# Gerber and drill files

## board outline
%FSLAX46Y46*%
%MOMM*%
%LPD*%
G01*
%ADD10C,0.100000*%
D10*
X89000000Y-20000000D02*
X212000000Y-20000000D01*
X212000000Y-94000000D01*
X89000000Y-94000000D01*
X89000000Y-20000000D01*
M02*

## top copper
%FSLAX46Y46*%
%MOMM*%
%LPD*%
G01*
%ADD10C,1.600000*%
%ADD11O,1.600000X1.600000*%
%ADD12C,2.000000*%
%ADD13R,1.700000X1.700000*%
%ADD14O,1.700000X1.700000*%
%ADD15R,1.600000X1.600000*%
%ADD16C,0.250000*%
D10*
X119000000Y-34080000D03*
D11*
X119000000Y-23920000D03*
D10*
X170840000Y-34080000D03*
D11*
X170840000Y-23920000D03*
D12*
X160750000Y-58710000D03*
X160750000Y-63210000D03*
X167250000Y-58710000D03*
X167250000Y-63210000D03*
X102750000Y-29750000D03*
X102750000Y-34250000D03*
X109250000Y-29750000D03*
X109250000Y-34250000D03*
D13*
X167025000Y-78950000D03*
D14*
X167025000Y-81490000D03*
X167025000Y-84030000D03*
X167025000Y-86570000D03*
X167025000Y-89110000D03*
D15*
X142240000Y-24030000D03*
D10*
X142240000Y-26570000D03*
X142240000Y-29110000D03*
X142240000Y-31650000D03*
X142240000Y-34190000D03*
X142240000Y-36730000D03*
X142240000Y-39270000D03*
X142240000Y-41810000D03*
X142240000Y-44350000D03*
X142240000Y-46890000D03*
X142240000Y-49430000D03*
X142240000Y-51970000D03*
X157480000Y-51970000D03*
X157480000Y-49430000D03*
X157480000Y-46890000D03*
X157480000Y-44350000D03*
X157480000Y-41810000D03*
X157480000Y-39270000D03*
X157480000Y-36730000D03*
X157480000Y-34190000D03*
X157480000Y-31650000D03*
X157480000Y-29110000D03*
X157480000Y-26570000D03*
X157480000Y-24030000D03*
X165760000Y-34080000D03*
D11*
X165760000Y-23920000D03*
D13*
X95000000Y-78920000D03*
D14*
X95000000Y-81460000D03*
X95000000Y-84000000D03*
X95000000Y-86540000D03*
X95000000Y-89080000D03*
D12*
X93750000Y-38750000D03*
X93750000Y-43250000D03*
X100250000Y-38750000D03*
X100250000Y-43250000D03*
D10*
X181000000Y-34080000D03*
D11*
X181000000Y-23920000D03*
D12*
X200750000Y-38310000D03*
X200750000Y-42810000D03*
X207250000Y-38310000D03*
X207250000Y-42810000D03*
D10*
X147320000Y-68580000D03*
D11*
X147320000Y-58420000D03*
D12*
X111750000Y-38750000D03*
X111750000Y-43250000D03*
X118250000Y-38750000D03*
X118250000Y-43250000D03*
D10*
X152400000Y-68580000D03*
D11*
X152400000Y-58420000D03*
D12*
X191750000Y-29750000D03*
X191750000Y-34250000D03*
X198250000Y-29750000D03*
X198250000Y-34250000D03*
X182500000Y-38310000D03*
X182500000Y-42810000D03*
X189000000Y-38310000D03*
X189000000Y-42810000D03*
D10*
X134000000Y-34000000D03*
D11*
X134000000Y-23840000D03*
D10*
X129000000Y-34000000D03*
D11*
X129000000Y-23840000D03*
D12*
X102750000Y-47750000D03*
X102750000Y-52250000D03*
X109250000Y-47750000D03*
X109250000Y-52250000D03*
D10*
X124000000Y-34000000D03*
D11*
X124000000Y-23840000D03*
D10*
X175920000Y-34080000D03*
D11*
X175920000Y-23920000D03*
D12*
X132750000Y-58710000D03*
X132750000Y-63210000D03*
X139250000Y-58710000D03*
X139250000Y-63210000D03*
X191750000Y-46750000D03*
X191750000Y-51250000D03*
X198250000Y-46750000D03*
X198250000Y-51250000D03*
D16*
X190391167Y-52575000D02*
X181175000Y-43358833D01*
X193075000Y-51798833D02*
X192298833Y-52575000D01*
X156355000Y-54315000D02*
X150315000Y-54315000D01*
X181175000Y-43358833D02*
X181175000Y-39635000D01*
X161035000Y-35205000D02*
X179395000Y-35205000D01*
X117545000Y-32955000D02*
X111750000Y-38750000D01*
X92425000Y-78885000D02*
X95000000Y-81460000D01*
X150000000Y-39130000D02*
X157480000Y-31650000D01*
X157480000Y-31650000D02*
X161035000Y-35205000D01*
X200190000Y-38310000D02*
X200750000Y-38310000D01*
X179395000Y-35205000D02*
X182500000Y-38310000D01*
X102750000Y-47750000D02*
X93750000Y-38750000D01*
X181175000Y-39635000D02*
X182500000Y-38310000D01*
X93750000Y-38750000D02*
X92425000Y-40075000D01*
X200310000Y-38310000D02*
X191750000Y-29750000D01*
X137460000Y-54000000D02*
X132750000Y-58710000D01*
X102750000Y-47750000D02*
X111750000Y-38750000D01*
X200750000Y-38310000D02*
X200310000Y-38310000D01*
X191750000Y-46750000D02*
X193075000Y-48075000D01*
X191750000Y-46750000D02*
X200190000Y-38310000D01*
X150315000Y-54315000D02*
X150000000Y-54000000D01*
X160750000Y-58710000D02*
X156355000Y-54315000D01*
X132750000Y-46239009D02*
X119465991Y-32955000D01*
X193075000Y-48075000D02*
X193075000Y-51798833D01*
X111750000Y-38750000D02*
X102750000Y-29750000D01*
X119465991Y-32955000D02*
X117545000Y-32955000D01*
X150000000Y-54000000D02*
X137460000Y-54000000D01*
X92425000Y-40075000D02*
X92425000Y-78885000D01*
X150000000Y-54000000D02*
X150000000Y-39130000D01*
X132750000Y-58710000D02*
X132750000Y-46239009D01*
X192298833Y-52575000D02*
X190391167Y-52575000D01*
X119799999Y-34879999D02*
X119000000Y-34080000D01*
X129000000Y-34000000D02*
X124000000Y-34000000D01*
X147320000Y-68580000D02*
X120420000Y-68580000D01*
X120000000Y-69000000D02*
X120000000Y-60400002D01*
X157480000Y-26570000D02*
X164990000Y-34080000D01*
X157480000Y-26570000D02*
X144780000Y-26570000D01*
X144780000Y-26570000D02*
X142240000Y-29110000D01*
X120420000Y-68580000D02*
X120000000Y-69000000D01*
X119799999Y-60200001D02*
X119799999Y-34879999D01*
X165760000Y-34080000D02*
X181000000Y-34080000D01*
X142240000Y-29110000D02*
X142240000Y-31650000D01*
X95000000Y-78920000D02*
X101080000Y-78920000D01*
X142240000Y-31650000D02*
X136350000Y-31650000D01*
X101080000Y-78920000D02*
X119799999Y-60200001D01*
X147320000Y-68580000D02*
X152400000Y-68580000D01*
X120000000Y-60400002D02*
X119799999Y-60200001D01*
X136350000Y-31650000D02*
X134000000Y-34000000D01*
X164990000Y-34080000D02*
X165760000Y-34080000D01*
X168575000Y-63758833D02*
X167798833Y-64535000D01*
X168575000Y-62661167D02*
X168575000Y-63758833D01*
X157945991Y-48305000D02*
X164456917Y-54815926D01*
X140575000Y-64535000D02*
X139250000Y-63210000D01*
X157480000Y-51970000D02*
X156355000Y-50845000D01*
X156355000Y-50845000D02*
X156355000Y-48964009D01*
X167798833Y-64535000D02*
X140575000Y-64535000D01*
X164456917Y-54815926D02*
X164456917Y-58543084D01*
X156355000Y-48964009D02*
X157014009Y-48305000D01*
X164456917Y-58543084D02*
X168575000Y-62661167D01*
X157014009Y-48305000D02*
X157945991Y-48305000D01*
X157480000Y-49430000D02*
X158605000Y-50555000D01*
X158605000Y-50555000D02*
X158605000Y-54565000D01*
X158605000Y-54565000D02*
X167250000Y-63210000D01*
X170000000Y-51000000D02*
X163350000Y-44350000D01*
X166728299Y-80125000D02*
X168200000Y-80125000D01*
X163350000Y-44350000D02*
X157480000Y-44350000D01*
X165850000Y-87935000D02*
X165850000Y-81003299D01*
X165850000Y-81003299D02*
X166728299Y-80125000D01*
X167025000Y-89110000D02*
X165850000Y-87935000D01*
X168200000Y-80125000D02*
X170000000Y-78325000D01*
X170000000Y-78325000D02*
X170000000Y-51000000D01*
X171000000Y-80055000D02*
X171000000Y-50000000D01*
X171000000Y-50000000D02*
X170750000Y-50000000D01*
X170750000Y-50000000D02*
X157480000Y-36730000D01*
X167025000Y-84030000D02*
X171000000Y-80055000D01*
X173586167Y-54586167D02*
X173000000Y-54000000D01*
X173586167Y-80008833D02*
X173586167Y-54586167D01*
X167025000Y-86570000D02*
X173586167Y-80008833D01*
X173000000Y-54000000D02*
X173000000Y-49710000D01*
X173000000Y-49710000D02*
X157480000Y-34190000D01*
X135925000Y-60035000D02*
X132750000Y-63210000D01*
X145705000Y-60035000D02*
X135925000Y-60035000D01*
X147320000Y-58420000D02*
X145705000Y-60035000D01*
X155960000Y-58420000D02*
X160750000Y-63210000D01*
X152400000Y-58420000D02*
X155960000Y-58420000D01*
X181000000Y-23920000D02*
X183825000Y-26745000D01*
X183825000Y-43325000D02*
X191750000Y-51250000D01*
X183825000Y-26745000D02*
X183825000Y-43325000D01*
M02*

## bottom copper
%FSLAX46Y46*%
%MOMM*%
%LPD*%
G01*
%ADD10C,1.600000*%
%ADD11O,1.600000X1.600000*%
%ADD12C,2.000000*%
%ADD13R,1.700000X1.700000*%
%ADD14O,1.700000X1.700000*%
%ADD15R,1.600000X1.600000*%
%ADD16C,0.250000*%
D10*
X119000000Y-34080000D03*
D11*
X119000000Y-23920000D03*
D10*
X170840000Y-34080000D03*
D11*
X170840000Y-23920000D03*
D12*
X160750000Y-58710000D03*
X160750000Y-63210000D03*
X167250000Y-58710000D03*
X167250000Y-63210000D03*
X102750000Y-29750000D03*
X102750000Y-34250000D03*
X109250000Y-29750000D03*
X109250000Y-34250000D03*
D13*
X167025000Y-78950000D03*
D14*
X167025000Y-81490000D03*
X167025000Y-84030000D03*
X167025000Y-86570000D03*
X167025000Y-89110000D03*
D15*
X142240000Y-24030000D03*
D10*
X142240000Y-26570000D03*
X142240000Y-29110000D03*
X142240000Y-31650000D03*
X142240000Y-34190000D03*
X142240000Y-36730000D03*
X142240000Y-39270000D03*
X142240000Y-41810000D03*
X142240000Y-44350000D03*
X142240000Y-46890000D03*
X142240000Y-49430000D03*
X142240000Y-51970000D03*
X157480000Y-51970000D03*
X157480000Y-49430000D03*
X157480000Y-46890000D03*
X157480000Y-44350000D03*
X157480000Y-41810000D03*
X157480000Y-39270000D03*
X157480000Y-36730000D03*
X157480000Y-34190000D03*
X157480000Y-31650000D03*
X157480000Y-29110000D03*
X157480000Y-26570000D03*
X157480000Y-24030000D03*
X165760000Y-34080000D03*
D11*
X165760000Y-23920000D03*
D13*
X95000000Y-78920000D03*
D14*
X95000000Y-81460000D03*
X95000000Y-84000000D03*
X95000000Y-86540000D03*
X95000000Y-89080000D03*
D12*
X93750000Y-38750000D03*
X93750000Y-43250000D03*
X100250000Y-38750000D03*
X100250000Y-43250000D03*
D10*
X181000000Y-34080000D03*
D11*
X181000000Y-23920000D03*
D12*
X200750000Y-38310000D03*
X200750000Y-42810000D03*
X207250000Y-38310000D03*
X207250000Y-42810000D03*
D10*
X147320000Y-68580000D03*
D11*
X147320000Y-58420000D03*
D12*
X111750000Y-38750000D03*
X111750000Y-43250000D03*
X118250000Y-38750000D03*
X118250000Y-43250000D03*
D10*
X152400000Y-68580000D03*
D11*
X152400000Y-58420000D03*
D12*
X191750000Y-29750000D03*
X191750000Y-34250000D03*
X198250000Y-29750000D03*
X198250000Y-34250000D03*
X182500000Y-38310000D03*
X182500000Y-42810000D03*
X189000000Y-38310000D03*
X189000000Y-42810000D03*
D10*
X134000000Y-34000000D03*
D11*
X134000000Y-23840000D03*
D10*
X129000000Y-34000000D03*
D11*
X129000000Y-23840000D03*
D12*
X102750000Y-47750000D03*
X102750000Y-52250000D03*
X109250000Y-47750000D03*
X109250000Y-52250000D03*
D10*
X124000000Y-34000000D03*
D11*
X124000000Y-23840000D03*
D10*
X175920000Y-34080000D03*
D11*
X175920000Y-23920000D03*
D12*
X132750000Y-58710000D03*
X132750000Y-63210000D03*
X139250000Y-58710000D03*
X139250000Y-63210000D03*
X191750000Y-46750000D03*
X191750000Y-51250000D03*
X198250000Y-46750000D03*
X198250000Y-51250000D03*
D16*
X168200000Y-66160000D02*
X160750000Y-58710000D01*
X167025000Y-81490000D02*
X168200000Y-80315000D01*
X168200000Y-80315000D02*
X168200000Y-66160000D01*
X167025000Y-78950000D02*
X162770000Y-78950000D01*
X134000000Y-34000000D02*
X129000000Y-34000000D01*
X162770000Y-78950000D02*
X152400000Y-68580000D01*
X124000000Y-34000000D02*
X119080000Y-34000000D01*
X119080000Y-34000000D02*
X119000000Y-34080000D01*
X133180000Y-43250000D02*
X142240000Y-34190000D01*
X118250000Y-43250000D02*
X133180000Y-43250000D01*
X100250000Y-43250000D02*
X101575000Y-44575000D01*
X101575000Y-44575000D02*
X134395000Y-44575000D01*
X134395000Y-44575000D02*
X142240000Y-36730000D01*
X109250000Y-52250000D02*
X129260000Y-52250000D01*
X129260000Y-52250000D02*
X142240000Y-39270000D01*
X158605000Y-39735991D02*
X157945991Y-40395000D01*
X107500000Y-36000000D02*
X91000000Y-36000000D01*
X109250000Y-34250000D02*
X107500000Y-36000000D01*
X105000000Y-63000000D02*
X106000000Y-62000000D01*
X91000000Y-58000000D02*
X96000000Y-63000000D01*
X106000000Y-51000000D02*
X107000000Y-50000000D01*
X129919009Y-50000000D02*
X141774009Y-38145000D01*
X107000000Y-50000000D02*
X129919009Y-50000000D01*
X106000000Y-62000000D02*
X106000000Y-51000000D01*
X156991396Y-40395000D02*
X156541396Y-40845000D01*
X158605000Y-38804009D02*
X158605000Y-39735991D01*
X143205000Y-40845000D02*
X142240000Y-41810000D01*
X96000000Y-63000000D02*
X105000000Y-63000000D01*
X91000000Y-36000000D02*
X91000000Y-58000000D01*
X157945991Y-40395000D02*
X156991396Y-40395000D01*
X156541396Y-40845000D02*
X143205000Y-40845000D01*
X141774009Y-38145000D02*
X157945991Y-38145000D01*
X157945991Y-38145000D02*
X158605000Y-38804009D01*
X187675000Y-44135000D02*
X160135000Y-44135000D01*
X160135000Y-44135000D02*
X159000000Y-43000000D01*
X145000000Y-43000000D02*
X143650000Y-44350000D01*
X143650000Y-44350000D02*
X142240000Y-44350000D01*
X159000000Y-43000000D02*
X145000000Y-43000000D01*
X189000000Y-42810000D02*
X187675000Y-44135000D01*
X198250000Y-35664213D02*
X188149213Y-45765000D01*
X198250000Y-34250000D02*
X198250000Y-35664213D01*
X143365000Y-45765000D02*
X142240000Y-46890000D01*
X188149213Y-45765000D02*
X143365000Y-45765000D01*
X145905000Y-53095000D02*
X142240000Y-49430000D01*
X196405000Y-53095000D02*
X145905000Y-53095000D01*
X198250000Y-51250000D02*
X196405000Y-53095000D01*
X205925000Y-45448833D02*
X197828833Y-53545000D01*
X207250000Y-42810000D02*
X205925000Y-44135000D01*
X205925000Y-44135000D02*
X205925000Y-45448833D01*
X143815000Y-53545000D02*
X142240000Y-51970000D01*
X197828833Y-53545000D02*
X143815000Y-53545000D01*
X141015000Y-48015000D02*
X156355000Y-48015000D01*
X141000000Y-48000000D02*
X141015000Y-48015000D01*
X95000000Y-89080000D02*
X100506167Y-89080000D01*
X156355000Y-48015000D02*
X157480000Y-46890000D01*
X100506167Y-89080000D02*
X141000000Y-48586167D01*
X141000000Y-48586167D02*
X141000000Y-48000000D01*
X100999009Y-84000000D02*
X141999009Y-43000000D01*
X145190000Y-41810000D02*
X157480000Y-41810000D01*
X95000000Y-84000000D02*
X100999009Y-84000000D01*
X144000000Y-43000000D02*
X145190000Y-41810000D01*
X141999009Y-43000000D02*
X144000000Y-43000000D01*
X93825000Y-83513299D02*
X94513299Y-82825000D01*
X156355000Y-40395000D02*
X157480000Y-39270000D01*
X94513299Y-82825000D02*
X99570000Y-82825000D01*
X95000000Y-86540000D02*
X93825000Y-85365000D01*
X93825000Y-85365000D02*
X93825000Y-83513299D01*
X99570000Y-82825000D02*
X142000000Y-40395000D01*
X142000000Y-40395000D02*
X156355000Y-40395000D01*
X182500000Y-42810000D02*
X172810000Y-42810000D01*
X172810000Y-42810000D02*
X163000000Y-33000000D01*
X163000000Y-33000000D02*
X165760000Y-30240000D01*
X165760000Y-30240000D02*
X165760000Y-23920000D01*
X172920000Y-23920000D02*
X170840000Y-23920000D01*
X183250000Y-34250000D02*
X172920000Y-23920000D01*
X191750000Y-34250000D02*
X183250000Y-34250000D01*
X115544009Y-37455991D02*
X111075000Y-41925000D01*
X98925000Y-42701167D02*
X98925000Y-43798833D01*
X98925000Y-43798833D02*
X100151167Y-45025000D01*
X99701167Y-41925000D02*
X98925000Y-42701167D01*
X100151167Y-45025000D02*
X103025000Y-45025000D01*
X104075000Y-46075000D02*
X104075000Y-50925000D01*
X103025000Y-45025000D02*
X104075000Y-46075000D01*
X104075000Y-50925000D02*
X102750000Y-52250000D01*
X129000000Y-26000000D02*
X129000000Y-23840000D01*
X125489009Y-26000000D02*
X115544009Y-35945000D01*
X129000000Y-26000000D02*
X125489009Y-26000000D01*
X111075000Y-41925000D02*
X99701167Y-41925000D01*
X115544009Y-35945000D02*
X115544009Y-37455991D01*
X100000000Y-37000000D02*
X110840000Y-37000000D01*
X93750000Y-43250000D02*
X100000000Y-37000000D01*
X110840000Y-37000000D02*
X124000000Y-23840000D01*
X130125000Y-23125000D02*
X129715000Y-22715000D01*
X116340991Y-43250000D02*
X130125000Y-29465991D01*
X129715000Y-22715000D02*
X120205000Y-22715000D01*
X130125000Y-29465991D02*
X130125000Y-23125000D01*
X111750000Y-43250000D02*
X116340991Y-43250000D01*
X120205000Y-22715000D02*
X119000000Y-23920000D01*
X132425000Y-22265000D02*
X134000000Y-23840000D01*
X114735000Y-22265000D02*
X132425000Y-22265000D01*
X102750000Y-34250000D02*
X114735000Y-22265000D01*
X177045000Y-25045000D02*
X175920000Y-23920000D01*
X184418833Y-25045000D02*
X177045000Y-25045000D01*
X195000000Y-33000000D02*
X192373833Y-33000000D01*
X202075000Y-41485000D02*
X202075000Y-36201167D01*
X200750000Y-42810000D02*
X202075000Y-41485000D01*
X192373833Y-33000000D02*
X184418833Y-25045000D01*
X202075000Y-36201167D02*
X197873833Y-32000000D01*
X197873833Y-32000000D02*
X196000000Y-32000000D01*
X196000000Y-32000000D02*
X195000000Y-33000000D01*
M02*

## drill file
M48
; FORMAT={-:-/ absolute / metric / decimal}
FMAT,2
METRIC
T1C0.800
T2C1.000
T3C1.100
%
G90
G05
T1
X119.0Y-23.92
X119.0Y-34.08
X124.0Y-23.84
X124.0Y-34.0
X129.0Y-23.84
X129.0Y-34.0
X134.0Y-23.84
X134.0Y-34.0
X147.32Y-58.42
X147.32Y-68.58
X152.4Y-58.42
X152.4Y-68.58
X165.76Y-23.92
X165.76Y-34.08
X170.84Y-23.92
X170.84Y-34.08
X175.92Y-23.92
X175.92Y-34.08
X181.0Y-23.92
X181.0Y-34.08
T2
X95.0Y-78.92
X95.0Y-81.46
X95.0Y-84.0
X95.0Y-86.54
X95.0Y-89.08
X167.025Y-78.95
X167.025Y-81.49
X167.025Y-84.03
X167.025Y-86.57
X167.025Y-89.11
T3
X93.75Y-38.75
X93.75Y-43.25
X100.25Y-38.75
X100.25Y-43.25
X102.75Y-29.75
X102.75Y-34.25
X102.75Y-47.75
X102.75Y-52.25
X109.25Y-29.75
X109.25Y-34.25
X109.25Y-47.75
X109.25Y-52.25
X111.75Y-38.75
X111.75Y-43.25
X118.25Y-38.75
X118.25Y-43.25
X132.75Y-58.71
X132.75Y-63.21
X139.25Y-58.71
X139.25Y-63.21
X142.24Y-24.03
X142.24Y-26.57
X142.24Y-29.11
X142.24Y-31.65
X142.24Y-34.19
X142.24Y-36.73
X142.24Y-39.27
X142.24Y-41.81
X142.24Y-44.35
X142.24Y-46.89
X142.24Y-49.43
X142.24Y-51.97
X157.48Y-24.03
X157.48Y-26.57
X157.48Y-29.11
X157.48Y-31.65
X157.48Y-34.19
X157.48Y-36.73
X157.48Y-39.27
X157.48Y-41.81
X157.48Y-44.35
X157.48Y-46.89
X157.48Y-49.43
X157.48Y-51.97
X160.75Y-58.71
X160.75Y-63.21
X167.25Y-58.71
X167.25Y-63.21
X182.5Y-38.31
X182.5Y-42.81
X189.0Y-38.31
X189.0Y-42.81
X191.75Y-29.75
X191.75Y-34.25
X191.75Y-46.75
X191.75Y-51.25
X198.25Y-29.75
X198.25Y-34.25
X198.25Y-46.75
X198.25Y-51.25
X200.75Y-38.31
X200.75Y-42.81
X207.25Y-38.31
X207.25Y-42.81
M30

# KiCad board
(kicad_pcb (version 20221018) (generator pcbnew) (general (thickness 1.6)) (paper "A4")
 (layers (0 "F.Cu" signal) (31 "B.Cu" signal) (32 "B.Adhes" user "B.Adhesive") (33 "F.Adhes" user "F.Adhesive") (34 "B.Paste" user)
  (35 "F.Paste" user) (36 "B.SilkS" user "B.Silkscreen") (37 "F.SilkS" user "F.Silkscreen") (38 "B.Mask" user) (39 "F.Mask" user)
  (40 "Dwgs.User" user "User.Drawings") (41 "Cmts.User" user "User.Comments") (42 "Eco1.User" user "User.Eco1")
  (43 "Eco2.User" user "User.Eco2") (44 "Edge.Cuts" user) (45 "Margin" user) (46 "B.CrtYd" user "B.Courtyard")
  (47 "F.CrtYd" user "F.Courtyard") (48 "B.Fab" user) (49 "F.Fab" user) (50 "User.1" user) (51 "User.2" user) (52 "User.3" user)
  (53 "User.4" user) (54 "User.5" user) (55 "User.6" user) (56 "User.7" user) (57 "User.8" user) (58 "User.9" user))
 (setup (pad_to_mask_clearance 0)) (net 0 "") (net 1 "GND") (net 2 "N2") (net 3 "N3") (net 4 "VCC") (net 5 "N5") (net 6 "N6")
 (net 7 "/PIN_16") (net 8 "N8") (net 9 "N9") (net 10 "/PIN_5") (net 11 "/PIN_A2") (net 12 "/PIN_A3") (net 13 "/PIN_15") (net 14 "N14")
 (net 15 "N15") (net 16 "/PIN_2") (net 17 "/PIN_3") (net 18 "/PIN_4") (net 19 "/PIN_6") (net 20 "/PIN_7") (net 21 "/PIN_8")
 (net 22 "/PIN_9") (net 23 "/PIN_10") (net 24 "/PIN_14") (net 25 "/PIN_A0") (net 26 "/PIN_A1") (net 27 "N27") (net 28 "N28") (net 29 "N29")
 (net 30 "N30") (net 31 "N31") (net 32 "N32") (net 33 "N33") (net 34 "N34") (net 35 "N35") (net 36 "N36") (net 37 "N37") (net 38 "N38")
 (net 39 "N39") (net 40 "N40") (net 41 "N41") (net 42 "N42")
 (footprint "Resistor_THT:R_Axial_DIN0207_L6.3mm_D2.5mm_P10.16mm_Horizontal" (layer "F.Cu") (at 119 34.08 90)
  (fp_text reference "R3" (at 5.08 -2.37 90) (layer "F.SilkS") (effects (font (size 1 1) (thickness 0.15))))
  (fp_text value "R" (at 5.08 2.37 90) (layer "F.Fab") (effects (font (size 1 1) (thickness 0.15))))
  (pad "1" thru_hole circle (at 0 0 90) (size 1.6 1.6) (drill 0.8) (layers "*.Cu" "*.Mask") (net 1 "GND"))
  (pad "2" thru_hole oval (at 10.16 0 90) (size 1.6 1.6) (drill 0.8) (layers "*.Cu" "*.Mask") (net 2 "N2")))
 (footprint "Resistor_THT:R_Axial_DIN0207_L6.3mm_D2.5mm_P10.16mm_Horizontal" (layer "F.Cu") (at 170.84 34.08 90)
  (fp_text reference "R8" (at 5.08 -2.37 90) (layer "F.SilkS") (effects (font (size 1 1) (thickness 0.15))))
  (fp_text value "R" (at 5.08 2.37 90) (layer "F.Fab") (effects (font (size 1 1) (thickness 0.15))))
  (pad "1" thru_hole circle (at 0 0 90) (size 1.6 1.6) (drill 0.8) (layers "*.Cu" "*.Mask") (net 1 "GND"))
  (pad "2" thru_hole oval (at 10.16 0 90) (size 1.6 1.6) (drill 0.8) (layers "*.Cu" "*.Mask") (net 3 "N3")))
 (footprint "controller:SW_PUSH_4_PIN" (layer "F.Cu") (at 160.75 58.71)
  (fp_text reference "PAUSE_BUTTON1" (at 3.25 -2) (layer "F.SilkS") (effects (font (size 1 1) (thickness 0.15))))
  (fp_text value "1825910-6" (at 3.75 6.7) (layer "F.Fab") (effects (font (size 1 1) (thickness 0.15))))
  (pad "1" thru_hole circle (at 0 0 90) (size 2 2) (drill 1.1) (layers "*.Cu" "*.Mask") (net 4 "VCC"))
  (pad "2" thru_hole circle (at 0 4.5 90) (size 2 2) (drill 1.1) (layers "*.Cu" "*.Mask") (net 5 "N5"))
  (pad "3" thru_hole circle (at 6.5 0 90) (size 2 2) (drill 1.1) (layers "*.Cu" "*.Mask") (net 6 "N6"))
  (pad "4" thru_hole circle (at 6.5 4.5 90) (size 2 2) (drill 1.1) (layers "*.Cu" "*.Mask") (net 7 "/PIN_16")))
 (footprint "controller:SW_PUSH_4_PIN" (layer "F.Cu") (at 102.75 29.75)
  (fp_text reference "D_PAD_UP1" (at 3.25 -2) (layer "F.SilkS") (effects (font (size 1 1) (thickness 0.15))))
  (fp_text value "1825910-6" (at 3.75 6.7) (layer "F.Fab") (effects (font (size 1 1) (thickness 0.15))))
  (pad "1" thru_hole circle (at 0 0 90) (size 2 2) (drill 1.1) (layers "*.Cu" "*.Mask") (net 4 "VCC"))
  (pad "2" thru_hole circle (at 0 4.5 90) (size 2 2) (drill 1.1) (layers "*.Cu" "*.Mask") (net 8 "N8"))
  (pad "3" thru_hole circle (at 6.5 0 90) (size 2 2) (drill 1.1) (layers "*.Cu" "*.Mask") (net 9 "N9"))
  (pad "4" thru_hole circle (at 6.5 4.5 90) (size 2 2) (drill 1.1) (layers "*.Cu" "*.Mask") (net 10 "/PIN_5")))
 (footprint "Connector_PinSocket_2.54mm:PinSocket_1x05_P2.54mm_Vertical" (layer "F.Cu") (at 167.025 78.95)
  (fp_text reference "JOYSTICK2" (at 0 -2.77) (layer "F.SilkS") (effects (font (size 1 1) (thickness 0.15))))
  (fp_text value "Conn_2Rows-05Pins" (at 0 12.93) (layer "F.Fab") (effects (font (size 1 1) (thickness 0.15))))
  (pad "1" thru_hole rect (at 0 0) (size 1.7 1.7) (drill 1) (layers "*.Cu" "*.Mask") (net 1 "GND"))
  (pad "2" thru_hole oval (at 0 2.54) (size 1.7 1.7) (drill 1) (layers "*.Cu" "*.Mask") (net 4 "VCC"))
  (pad "3" thru_hole oval (at 0 5.08) (size 1.7 1.7) (drill 1) (layers "*.Cu" "*.Mask") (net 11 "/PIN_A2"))
  (pad "4" thru_hole oval (at 0 7.62) (size 1.7 1.7) (drill 1) (layers "*.Cu" "*.Mask") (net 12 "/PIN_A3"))
  (pad "5" thru_hole oval (at 0 10.16) (size 1.7 1.7) (drill 1) (layers "*.Cu" "*.Mask") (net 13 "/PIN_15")))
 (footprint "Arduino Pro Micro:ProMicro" (layer "F.Cu") (at 149.86 38 -90)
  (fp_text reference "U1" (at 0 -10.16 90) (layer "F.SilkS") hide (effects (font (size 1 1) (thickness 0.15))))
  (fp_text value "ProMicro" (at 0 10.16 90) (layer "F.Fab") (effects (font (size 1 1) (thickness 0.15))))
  (pad "1" thru_hole rect (at -13.97 7.62 270) (size 1.6 1.6) (drill 1.1) (layers "*.Cu" "*.Mask" "F.SilkS") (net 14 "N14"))
  (pad "2" thru_hole circle (at -11.43 7.62 270) (size 1.6 1.6) (drill 1.1) (layers "*.Cu" "*.Mask" "F.SilkS") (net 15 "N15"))
  (pad "3" thru_hole circle (at -8.89 7.62 270) (size 1.6 1.6) (drill 1.1) (layers "*.Cu" "*.Mask" "F.SilkS") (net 1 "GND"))
  (pad "4" thru_hole circle (at -6.35 7.62 270) (size 1.6 1.6) (drill 1.1) (layers "*.Cu" "*.Mask" "F.SilkS") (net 1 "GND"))
  (pad "5" thru_hole circle (at -3.81 7.62 270) (size 1.6 1.6) (drill 1.1) (layers "*.Cu" "*.Mask" "F.SilkS") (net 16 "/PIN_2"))
  (pad "6" thru_hole circle (at -1.27 7.62 270) (size 1.6 1.6) (drill 1.1) (layers "*.Cu" "*.Mask" "F.SilkS") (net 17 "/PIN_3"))
  (pad "7" thru_hole circle (at 1.27 7.62 270) (size 1.6 1.6) (drill 1.1) (layers "*.Cu" "*.Mask" "F.SilkS") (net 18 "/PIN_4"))
  (pad "8" thru_hole circle (at 3.81 7.62 270) (size 1.6 1.6) (drill 1.1) (layers "*.Cu" "*.Mask" "F.SilkS") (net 10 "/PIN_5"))
  (pad "9" thru_hole circle (at 6.35 7.62 270) (size 1.6 1.6) (drill 1.1) (layers "*.Cu" "*.Mask" "F.SilkS") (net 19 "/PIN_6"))
  (pad "10" thru_hole circle (at 8.89 7.62 270) (size 1.6 1.6) (drill 1.1) (layers "*.Cu" "*.Mask" "F.SilkS") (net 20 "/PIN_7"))
  (pad "11" thru_hole circle (at 11.43 7.62 270) (size 1.6 1.6) (drill 1.1) (layers "*.Cu" "*.Mask" "F.SilkS") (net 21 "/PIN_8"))
  (pad "12" thru_hole circle (at 13.97 7.62 270) (size 1.6 1.6) (drill 1.1) (layers "*.Cu" "*.Mask" "F.SilkS") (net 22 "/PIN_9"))
  (pad "13" thru_hole circle (at 13.97 -7.62 270) (size 1.6 1.6) (drill 1.1) (layers "*.Cu" "*.Mask" "F.SilkS") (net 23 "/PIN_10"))
  (pad "14" thru_hole circle (at 11.43 -7.62 270) (size 1.6 1.6) (drill 1.1) (layers "*.Cu" "*.Mask" "F.SilkS") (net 7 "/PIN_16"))
  (pad "15" thru_hole circle (at 8.89 -7.62 270) (size 1.6 1.6) (drill 1.1) (layers "*.Cu" "*.Mask" "F.SilkS") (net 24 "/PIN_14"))
  (pad "16" thru_hole circle (at 6.35 -7.62 270) (size 1.6 1.6) (drill 1.1) (layers "*.Cu" "*.Mask" "F.SilkS") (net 13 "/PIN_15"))
  (pad "17" thru_hole circle (at 3.81 -7.62 270) (size 1.6 1.6) (drill 1.1) (layers "*.Cu" "*.Mask" "F.SilkS") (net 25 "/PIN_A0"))
  (pad "18" thru_hole circle (at 1.27 -7.62 270) (size 1.6 1.6) (drill 1.1) (layers "*.Cu" "*.Mask" "F.SilkS") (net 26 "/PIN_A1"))
  (pad "19" thru_hole circle (at -1.27 -7.62 270) (size 1.6 1.6) (drill 1.1) (layers "*.Cu" "*.Mask" "F.SilkS") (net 11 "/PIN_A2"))
  (pad "20" thru_hole circle (at -3.81 -7.62 270) (size 1.6 1.6) (drill 1.1) (layers "*.Cu" "*.Mask" "F.SilkS") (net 12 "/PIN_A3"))
  (pad "21" thru_hole circle (at -6.35 -7.62 270) (size 1.6 1.6) (drill 1.1) (layers "*.Cu" "*.Mask" "F.SilkS") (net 4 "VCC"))
  (pad "22" thru_hole circle (at -8.89 -7.62 270) (size 1.6 1.6) (drill 1.1) (layers "*.Cu" "*.Mask" "F.SilkS") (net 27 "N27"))
  (pad "23" thru_hole circle (at -11.43 -7.62 270) (size 1.6 1.6) (drill 1.1) (layers "*.Cu" "*.Mask" "F.SilkS") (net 1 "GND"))
  (pad "24" thru_hole circle (at -13.97 -7.62 270) (size 1.6 1.6) (drill 1.1) (layers "*.Cu" "*.Mask" "F.SilkS") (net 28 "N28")))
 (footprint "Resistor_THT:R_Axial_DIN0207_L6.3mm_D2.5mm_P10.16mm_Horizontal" (layer "F.Cu") (at 165.76 34.08 90)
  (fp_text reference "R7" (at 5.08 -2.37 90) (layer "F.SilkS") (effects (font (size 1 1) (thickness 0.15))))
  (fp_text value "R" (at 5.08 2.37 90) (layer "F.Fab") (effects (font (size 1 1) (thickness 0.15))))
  (pad "1" thru_hole circle (at 0 0 90) (size 1.6 1.6) (drill 0.8) (layers "*.Cu" "*.Mask") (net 1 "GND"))
  (pad "2" thru_hole oval (at 10.16 0 90) (size 1.6 1.6) (drill 0.8) (layers "*.Cu" "*.Mask") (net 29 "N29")))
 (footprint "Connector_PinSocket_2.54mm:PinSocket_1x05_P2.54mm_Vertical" (layer "F.Cu") (at 95 78.92)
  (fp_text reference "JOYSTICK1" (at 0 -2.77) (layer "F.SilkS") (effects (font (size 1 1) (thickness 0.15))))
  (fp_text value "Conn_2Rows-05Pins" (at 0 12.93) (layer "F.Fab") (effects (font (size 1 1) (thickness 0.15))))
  (pad "1" thru_hole rect (at 0 0) (size 1.7 1.7) (drill 1) (layers "*.Cu" "*.Mask") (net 1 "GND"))
  (pad "2" thru_hole oval (at 0 2.54) (size 1.7 1.7) (drill 1) (layers "*.Cu" "*.Mask") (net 4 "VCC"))
  (pad "3" thru_hole oval (at 0 5.08) (size 1.7 1.7) (drill 1) (layers "*.Cu" "*.Mask") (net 25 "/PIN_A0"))
  (pad "4" thru_hole oval (at 0 7.62) (size 1.7 1.7) (drill 1) (layers "*.Cu" "*.Mask") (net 26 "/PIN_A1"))
  (pad "5" thru_hole oval (at 0 10.16) (size 1.7 1.7) (drill 1) (layers "*.Cu" "*.Mask") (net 24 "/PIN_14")))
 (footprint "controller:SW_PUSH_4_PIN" (layer "F.Cu") (at 93.75 38.75)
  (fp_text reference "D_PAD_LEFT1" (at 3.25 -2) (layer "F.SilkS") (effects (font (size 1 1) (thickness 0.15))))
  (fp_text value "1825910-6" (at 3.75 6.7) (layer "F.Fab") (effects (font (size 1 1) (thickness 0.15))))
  (pad "1" thru_hole circle (at 0 0 90) (size 2 2) (drill 1.1) (layers "*.Cu" "*.Mask") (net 4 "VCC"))
  (pad "2" thru_hole circle (at 0 4.5 90) (size 2 2) (drill 1.1) (layers "*.Cu" "*.Mask") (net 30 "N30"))
  (pad "3" thru_hole circle (at 6.5 0 90) (size 2 2) (drill 1.1) (layers "*.Cu" "*.Mask") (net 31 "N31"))
  (pad "4" thru_hole circle (at 6.5 4.5 90) (size 2 2) (drill 1.1) (layers "*.Cu" "*.Mask") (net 17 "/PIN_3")))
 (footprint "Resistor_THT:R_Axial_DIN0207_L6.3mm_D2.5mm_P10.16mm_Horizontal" (layer "F.Cu") (at 181 34.08 90)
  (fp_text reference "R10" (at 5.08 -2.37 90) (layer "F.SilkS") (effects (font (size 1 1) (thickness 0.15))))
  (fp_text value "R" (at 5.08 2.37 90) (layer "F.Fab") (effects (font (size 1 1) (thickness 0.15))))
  (pad "1" thru_hole circle (at 0 0 90) (size 1.6 1.6) (drill 0.8) (layers "*.Cu" "*.Mask") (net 1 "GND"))
  (pad "2" thru_hole oval (at 10.16 0 90) (size 1.6 1.6) (drill 0.8) (layers "*.Cu" "*.Mask") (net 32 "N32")))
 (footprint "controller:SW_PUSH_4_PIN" (layer "F.Cu") (at 200.75 38.31)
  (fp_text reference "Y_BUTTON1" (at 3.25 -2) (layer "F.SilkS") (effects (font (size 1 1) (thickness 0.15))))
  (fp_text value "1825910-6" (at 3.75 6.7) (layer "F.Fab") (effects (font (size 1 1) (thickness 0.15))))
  (pad "1" thru_hole circle (at 0 0 90) (size 2 2) (drill 1.1) (layers "*.Cu" "*.Mask") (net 4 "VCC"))
  (pad "2" thru_hole circle (at 0 4.5 90) (size 2 2) (drill 1.1) (layers "*.Cu" "*.Mask") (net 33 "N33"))
  (pad "3" thru_hole circle (at 6.5 0 90) (size 2 2) (drill 1.1) (layers "*.Cu" "*.Mask") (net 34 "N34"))
  (pad "4" thru_hole circle (at 6.5 4.5 90) (size 2 2) (drill 1.1) (layers "*.Cu" "*.Mask") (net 22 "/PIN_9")))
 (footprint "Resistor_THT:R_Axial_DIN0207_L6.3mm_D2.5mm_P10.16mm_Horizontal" (layer "F.Cu") (at 147.32 68.58 90)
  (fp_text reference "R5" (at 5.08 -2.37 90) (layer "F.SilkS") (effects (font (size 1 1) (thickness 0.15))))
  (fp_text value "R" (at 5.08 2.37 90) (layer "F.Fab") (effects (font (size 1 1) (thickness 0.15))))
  (pad "1" thru_hole circle (at 0 0 90) (size 1.6 1.6) (drill 0.8) (layers "*.Cu" "*.Mask") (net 1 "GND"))
  (pad "2" thru_hole oval (at 10.16 0 90) (size 1.6 1.6) (drill 0.8) (layers "*.Cu" "*.Mask") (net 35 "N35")))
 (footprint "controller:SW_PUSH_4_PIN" (layer "F.Cu") (at 111.75 38.75)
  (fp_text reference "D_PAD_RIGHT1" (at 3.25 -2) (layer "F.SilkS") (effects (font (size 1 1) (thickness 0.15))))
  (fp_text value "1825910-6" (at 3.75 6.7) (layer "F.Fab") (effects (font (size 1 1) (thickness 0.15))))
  (pad "1" thru_hole circle (at 0 0 90) (size 2 2) (drill 1.1) (layers "*.Cu" "*.Mask") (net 4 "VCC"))
  (pad "2" thru_hole circle (at 0 4.5 90) (size 2 2) (drill 1.1) (layers "*.Cu" "*.Mask") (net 2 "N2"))
  (pad "3" thru_hole circle (at 6.5 0 90) (size 2 2) (drill 1.1) (layers "*.Cu" "*.Mask") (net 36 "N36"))
  (pad "4" thru_hole circle (at 6.5 4.5 90) (size 2 2) (drill 1.1) (layers "*.Cu" "*.Mask") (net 16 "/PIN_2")))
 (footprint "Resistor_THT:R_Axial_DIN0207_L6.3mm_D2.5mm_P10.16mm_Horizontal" (layer "F.Cu") (at 152.4 68.58 90)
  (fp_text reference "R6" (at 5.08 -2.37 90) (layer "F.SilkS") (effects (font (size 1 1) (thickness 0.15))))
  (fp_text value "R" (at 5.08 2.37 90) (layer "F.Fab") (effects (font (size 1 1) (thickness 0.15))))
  (pad "1" thru_hole circle (at 0 0 90) (size 1.6 1.6) (drill 0.8) (layers "*.Cu" "*.Mask") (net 1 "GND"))
  (pad "2" thru_hole oval (at 10.16 0 90) (size 1.6 1.6) (drill 0.8) (layers "*.Cu" "*.Mask") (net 5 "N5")))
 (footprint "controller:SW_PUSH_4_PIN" (layer "F.Cu") (at 191.75 29.75)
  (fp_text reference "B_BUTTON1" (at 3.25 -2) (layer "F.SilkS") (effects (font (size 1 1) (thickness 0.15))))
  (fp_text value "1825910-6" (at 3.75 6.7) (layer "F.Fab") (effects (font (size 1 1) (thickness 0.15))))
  (pad "1" thru_hole circle (at 0 0 90) (size 2 2) (drill 1.1) (layers "*.Cu" "*.Mask") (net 4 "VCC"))
  (pad "2" thru_hole circle (at 0 4.5 90) (size 2 2) (drill 1.1) (layers "*.Cu" "*.Mask") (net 3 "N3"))
  (pad "3" thru_hole circle (at 6.5 0 90) (size 2 2) (drill 1.1) (layers "*.Cu" "*.Mask") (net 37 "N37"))
  (pad "4" thru_hole circle (at 6.5 4.5 90) (size 2 2) (drill 1.1) (layers "*.Cu" "*.Mask") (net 20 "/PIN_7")))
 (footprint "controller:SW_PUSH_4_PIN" (layer "F.Cu") (at 182.5 38.31)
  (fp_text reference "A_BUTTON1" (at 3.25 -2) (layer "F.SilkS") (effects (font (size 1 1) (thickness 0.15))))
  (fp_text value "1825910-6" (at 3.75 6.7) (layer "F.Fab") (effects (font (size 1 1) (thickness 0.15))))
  (pad "1" thru_hole circle (at 0 0 90) (size 2 2) (drill 1.1) (layers "*.Cu" "*.Mask") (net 4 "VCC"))
  (pad "2" thru_hole circle (at 0 4.5 90) (size 2 2) (drill 1.1) (layers "*.Cu" "*.Mask") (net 29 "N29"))
  (pad "3" thru_hole circle (at 6.5 0 90) (size 2 2) (drill 1.1) (layers "*.Cu" "*.Mask") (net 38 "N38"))
  (pad "4" thru_hole circle (at 6.5 4.5 90) (size 2 2) (drill 1.1) (layers "*.Cu" "*.Mask") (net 19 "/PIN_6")))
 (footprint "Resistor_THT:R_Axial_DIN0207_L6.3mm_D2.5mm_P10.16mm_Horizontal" (layer "F.Cu") (at 134 34 90)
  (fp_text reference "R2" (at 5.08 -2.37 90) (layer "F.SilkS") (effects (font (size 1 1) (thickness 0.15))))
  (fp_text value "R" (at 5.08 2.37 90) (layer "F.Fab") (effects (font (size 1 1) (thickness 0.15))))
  (pad "1" thru_hole circle (at 0 0 90) (size 1.6 1.6) (drill 0.8) (layers "*.Cu" "*.Mask") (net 1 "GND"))
  (pad "2" thru_hole oval (at 10.16 0 90) (size 1.6 1.6) (drill 0.8) (layers "*.Cu" "*.Mask") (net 8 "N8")))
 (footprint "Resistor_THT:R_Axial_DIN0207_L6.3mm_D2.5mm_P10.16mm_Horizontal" (layer "F.Cu") (at 129 34 90)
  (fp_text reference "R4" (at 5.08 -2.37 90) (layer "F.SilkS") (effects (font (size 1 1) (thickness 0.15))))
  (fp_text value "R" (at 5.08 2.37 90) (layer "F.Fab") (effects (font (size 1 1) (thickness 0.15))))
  (pad "1" thru_hole circle (at 0 0 90) (size 1.6 1.6) (drill 0.8) (layers "*.Cu" "*.Mask") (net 1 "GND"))
  (pad "2" thru_hole oval (at 10.16 0 90) (size 1.6 1.6) (drill 0.8) (layers "*.Cu" "*.Mask") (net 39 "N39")))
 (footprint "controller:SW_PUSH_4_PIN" (layer "F.Cu") (at 102.75 47.75)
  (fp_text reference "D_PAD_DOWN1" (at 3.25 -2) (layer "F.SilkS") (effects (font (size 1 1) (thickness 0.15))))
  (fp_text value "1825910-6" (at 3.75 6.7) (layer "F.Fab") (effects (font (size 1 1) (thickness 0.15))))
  (pad "1" thru_hole circle (at 0 0 90) (size 2 2) (drill 1.1) (layers "*.Cu" "*.Mask") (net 4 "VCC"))
  (pad "2" thru_hole circle (at 0 4.5 90) (size 2 2) (drill 1.1) (layers "*.Cu" "*.Mask") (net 39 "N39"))
  (pad "3" thru_hole circle (at 6.5 0 90) (size 2 2) (drill 1.1) (layers "*.Cu" "*.Mask") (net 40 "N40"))
  (pad "4" thru_hole circle (at 6.5 4.5 90) (size 2 2) (drill 1.1) (layers "*.Cu" "*.Mask") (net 18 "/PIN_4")))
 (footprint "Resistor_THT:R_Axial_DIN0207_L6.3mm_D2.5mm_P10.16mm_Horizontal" (layer "F.Cu") (at 124 34 90)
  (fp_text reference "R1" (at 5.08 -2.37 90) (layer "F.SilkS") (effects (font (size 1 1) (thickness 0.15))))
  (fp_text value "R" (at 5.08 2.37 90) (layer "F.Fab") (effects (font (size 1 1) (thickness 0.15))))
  (pad "1" thru_hole circle (at 0 0 90) (size 1.6 1.6) (drill 0.8) (layers "*.Cu" "*.Mask") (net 1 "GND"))
  (pad "2" thru_hole oval (at 10.16 0 90) (size 1.6 1.6) (drill 0.8) (layers "*.Cu" "*.Mask") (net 30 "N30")))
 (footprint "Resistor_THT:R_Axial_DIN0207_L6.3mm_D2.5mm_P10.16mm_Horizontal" (layer "F.Cu") (at 175.92 34.08 90)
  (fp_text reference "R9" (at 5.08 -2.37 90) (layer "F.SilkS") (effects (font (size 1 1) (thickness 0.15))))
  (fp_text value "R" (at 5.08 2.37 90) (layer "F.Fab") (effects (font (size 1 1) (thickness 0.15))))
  (pad "1" thru_hole circle (at 0 0 90) (size 1.6 1.6) (drill 0.8) (layers "*.Cu" "*.Mask") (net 1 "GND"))
  (pad "2" thru_hole oval (at 10.16 0 90) (size 1.6 1.6) (drill 0.8) (layers "*.Cu" "*.Mask") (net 33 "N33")))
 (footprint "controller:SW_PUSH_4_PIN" (layer "F.Cu") (at 132.75 58.71)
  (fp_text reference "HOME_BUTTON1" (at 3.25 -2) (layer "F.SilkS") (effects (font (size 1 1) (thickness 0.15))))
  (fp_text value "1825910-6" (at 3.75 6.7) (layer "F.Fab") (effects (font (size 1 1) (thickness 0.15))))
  (pad "1" thru_hole circle (at 0 0 90) (size 2 2) (drill 1.1) (layers "*.Cu" "*.Mask") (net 4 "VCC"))
  (pad "2" thru_hole circle (at 0 4.5 90) (size 2 2) (drill 1.1) (layers "*.Cu" "*.Mask") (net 35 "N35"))
  (pad "3" thru_hole circle (at 6.5 0 90) (size 2 2) (drill 1.1) (layers "*.Cu" "*.Mask") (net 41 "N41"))
  (pad "4" thru_hole circle (at 6.5 4.5 90) (size 2 2) (drill 1.1) (layers "*.Cu" "*.Mask") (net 23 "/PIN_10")))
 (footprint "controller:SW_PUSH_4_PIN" (layer "F.Cu") (at 191.75 46.75)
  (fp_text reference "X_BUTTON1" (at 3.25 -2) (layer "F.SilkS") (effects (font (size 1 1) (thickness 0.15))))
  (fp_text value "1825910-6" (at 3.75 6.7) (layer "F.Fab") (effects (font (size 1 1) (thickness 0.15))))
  (pad "1" thru_hole circle (at 0 0 90) (size 2 2) (drill 1.1) (layers "*.Cu" "*.Mask") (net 4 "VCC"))
  (pad "2" thru_hole circle (at 0 4.5 90) (size 2 2) (drill 1.1) (layers "*.Cu" "*.Mask") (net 32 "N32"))
  (pad "3" thru_hole circle (at 6.5 0 90) (size 2 2) (drill 1.1) (layers "*.Cu" "*.Mask") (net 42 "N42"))
  (pad "4" thru_hole circle (at 6.5 4.5 90) (size 2 2) (drill 1.1) (layers "*.Cu" "*.Mask") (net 21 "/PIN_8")))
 (gr_rect (start 89 20) (end 212 94) (stroke (width 0.1) (type default)) (fill none) (layer "Edge.Cuts"))
 (segment (start 190.391167 52.575) (end 181.175 43.358833) (width 0.25) (layer "F.Cu") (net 4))
 (segment (start 193.075 51.798833) (end 192.298833 52.575) (width 0.25) (layer "F.Cu") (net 4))
 (segment (start 156.355 54.315) (end 150.315 54.315) (width 0.25) (layer "F.Cu") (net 4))
 (segment (start 181.175 43.358833) (end 181.175 39.635) (width 0.25) (layer "F.Cu") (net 4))
 (segment (start 161.035 35.205) (end 179.395 35.205) (width 0.25) (layer "F.Cu") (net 4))
 (segment (start 117.545 32.955) (end 111.75 38.75) (width 0.25) (layer "F.Cu") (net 4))
 (segment (start 92.425 78.885) (end 95 81.46) (width 0.25) (layer "F.Cu") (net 4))
 (segment (start 150 39.13) (end 157.48 31.65) (width 0.25) (layer "F.Cu") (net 4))
 (segment (start 157.48 31.65) (end 161.035 35.205) (width 0.25) (layer "F.Cu") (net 4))
 (segment (start 200.19 38.31) (end 200.75 38.31) (width 0.25) (layer "F.Cu") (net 4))
 (segment (start 179.395 35.205) (end 182.5 38.31) (width 0.25) (layer "F.Cu") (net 4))
 (segment (start 102.75 47.75) (end 93.75 38.75) (width 0.25) (layer "F.Cu") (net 4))
 (segment (start 181.175 39.635) (end 182.5 38.31) (width 0.25) (layer "F.Cu") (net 4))
 (segment (start 93.75 38.75) (end 92.425 40.075) (width 0.25) (layer "F.Cu") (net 4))
 (segment (start 200.31 38.31) (end 191.75 29.75) (width 0.25) (layer "F.Cu") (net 4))
 (segment (start 137.46 54) (end 132.75 58.71) (width 0.25) (layer "F.Cu") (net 4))
 (segment (start 102.75 47.75) (end 111.75 38.75) (width 0.25) (layer "F.Cu") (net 4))
 (segment (start 200.75 38.31) (end 200.31 38.31) (width 0.25) (layer "F.Cu") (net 4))
 (segment (start 191.75 46.75) (end 193.075 48.075) (width 0.25) (layer "F.Cu") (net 4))
 (segment (start 191.75 46.75) (end 200.19 38.31) (width 0.25) (layer "F.Cu") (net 4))
 (segment (start 150.315 54.315) (end 150 54) (width 0.25) (layer "F.Cu") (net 4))
 (segment (start 160.75 58.71) (end 156.355 54.315) (width 0.25) (layer "F.Cu") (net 4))
 (segment (start 132.75 46.239009) (end 119.465991 32.955) (width 0.25) (layer "F.Cu") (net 4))
 (segment (start 193.075 48.075) (end 193.075 51.798833) (width 0.25) (layer "F.Cu") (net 4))
 (segment (start 111.75 38.75) (end 102.75 29.75) (width 0.25) (layer "F.Cu") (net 4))
 (segment (start 119.465991 32.955) (end 117.545 32.955) (width 0.25) (layer "F.Cu") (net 4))
 (segment (start 150 54) (end 137.46 54) (width 0.25) (layer "F.Cu") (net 4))
 (segment (start 92.425 40.075) (end 92.425 78.885) (width 0.25) (layer "F.Cu") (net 4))
 (segment (start 150 54) (end 150 39.13) (width 0.25) (layer "F.Cu") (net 4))
 (segment (start 132.75 58.71) (end 132.75 46.239009) (width 0.25) (layer "F.Cu") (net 4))
 (segment (start 192.298833 52.575) (end 190.391167 52.575) (width 0.25) (layer "F.Cu") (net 4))
 (segment (start 168.2 66.16) (end 160.75 58.71) (width 0.25) (layer "B.Cu") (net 4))
 (segment (start 167.025 81.49) (end 168.2 80.315) (width 0.25) (layer "B.Cu") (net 4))
 (segment (start 168.2 80.315) (end 168.2 66.16) (width 0.25) (layer "B.Cu") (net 4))
 (segment (start 119.799999 34.879999) (end 119 34.08) (width 0.25) (layer "F.Cu") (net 1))
 (segment (start 129 34) (end 124 34) (width 0.25) (layer "F.Cu") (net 1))
 (segment (start 147.32 68.58) (end 120.42 68.58) (width 0.25) (layer "F.Cu") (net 1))
 (segment (start 120 69) (end 120 60.400002) (width 0.25) (layer "F.Cu") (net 1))
 (segment (start 157.48 26.57) (end 164.99 34.08) (width 0.25) (layer "F.Cu") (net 1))
 (segment (start 157.48 26.57) (end 144.78 26.57) (width 0.25) (layer "F.Cu") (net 1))
 (segment (start 144.78 26.57) (end 142.24 29.11) (width 0.25) (layer "F.Cu") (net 1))
 (segment (start 120.42 68.58) (end 120 69) (width 0.25) (layer "F.Cu") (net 1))
 (segment (start 119.799999 60.200001) (end 119.799999 34.879999) (width 0.25) (layer "F.Cu") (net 1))
 (segment (start 165.76 34.08) (end 181 34.08) (width 0.25) (layer "F.Cu") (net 1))
 (segment (start 142.24 29.11) (end 142.24 31.65) (width 0.25) (layer "F.Cu") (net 1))
 (segment (start 95 78.92) (end 101.08 78.92) (width 0.25) (layer "F.Cu") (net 1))
 (segment (start 142.24 31.65) (end 136.35 31.65) (width 0.25) (layer "F.Cu") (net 1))
 (segment (start 101.08 78.92) (end 119.799999 60.200001) (width 0.25) (layer "F.Cu") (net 1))
 (segment (start 147.32 68.58) (end 152.4 68.58) (width 0.25) (layer "F.Cu") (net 1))
 (segment (start 120 60.400002) (end 119.799999 60.200001) (width 0.25) (layer "F.Cu") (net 1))
 (segment (start 136.35 31.65) (end 134 34) (width 0.25) (layer "F.Cu") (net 1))
 (segment (start 164.99 34.08) (end 165.76 34.08) (width 0.25) (layer "F.Cu") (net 1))
 (segment (start 167.025 78.95) (end 162.77 78.95) (width 0.25) (layer "B.Cu") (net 1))
 (segment (start 134 34) (end 129 34) (width 0.25) (layer "B.Cu") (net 1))
 (segment (start 162.77 78.95) (end 152.4 68.58) (width 0.25) (layer "B.Cu") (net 1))
 (segment (start 124 34) (end 119.08 34) (width 0.25) (layer "B.Cu") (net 1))
 (segment (start 119.08 34) (end 119 34.08) (width 0.25) (layer "B.Cu") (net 1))
 (segment (start 133.18 43.25) (end 142.24 34.19) (width 0.25) (layer "B.Cu") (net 16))
 (segment (start 118.25 43.25) (end 133.18 43.25) (width 0.25) (layer "B.Cu") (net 16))
 (segment (start 100.25 43.25) (end 101.575 44.575) (width 0.25) (layer "B.Cu") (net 17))
 (segment (start 101.575 44.575) (end 134.395 44.575) (width 0.25) (layer "B.Cu") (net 17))
 (segment (start 134.395 44.575) (end 142.24 36.73) (width 0.25) (layer "B.Cu") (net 17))
 (segment (start 109.25 52.25) (end 129.26 52.25) (width 0.25) (layer "B.Cu") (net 18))
 (segment (start 129.26 52.25) (end 142.24 39.27) (width 0.25) (layer "B.Cu") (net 18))
 (segment (start 158.605 39.735991) (end 157.945991 40.395) (width 0.25) (layer "B.Cu") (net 10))
 (segment (start 107.5 36) (end 91 36) (width 0.25) (layer "B.Cu") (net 10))
 (segment (start 109.25 34.25) (end 107.5 36) (width 0.25) (layer "B.Cu") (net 10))
 (segment (start 105 63) (end 106 62) (width 0.25) (layer "B.Cu") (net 10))
 (segment (start 91 58) (end 96 63) (width 0.25) (layer "B.Cu") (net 10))
 (segment (start 106 51) (end 107 50) (width 0.25) (layer "B.Cu") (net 10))
 (segment (start 129.919009 50) (end 141.774009 38.145) (width 0.25) (layer "B.Cu") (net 10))
 (segment (start 107 50) (end 129.919009 50) (width 0.25) (layer "B.Cu") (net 10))
 (segment (start 106 62) (end 106 51) (width 0.25) (layer "B.Cu") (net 10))
 (segment (start 156.991396 40.395) (end 156.541396 40.845) (width 0.25) (layer "B.Cu") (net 10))
 (segment (start 158.605 38.804009) (end 158.605 39.735991) (width 0.25) (layer "B.Cu") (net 10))
 (segment (start 143.205 40.845) (end 142.24 41.81) (width 0.25) (layer "B.Cu") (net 10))
 (segment (start 96 63) (end 105 63) (width 0.25) (layer "B.Cu") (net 10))
 (segment (start 91 36) (end 91 58) (width 0.25) (layer "B.Cu") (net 10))
 (segment (start 157.945991 40.395) (end 156.991396 40.395) (width 0.25) (layer "B.Cu") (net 10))
 (segment (start 156.541396 40.845) (end 143.205 40.845) (width 0.25) (layer "B.Cu") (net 10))
 (segment (start 141.774009 38.145) (end 157.945991 38.145) (width 0.25) (layer "B.Cu") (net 10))
 (segment (start 157.945991 38.145) (end 158.605 38.804009) (width 0.25) (layer "B.Cu") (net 10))
 (segment (start 187.675 44.135) (end 160.135 44.135) (width 0.25) (layer "B.Cu") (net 19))
 (segment (start 160.135 44.135) (end 159 43) (width 0.25) (layer "B.Cu") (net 19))
 (segment (start 145 43) (end 143.65 44.35) (width 0.25) (layer "B.Cu") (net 19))
 (segment (start 143.65 44.35) (end 142.24 44.35) (width 0.25) (layer "B.Cu") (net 19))
 (segment (start 159 43) (end 145 43) (width 0.25) (layer "B.Cu") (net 19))
 (segment (start 189 42.81) (end 187.675 44.135) (width 0.25) (layer "B.Cu") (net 19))
 (segment (start 198.25 35.664213) (end 188.149213 45.765) (width 0.25) (layer "B.Cu") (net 20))
 (segment (start 198.25 34.25) (end 198.25 35.664213) (width 0.25) (layer "B.Cu") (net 20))
 (segment (start 143.365 45.765) (end 142.24 46.89) (width 0.25) (layer "B.Cu") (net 20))
 (segment (start 188.149213 45.765) (end 143.365 45.765) (width 0.25) (layer "B.Cu") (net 20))
 (segment (start 145.905 53.095) (end 142.24 49.43) (width 0.25) (layer "B.Cu") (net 21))
 (segment (start 196.405 53.095) (end 145.905 53.095) (width 0.25) (layer "B.Cu") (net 21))
 (segment (start 198.25 51.25) (end 196.405 53.095) (width 0.25) (layer "B.Cu") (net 21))
 (segment (start 205.925 45.448833) (end 197.828833 53.545) (width 0.25) (layer "B.Cu") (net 22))
 (segment (start 207.25 42.81) (end 205.925 44.135) (width 0.25) (layer "B.Cu") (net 22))
 (segment (start 205.925 44.135) (end 205.925 45.448833) (width 0.25) (layer "B.Cu") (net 22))
 (segment (start 143.815 53.545) (end 142.24 51.97) (width 0.25) (layer "B.Cu") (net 22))
 (segment (start 197.828833 53.545) (end 143.815 53.545) (width 0.25) (layer "B.Cu") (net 22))
 (segment (start 168.575 63.758833) (end 167.798833 64.535) (width 0.25) (layer "F.Cu") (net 23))
 (segment (start 168.575 62.661167) (end 168.575 63.758833) (width 0.25) (layer "F.Cu") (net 23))
 (segment (start 157.945991 48.305) (end 164.456917 54.815926) (width 0.25) (layer "F.Cu") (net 23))
 (segment (start 140.575 64.535) (end 139.25 63.21) (width 0.25) (layer "F.Cu") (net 23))
 (segment (start 157.48 51.97) (end 156.355 50.845) (width 0.25) (layer "F.Cu") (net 23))
 (segment (start 156.355 50.845) (end 156.355 48.964009) (width 0.25) (layer "F.Cu") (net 23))
 (segment (start 167.798833 64.535) (end 140.575 64.535) (width 0.25) (layer "F.Cu") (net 23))
 (segment (start 164.456917 54.815926) (end 164.456917 58.543084) (width 0.25) (layer "F.Cu") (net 23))
 (segment (start 156.355 48.964009) (end 157.014009 48.305) (width 0.25) (layer "F.Cu") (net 23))
 (segment (start 164.456917 58.543084) (end 168.575 62.661167) (width 0.25) (layer "F.Cu") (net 23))
 (segment (start 157.014009 48.305) (end 157.945991 48.305) (width 0.25) (layer "F.Cu") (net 23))
 (segment (start 157.48 49.43) (end 158.605 50.555) (width 0.25) (layer "F.Cu") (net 7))
 (segment (start 158.605 50.555) (end 158.605 54.565) (width 0.25) (layer "F.Cu") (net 7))
 (segment (start 158.605 54.565) (end 167.25 63.21) (width 0.25) (layer "F.Cu") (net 7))
 (segment (start 141.015 48.015) (end 156.355 48.015) (width 0.25) (layer "B.Cu") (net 24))
 (segment (start 141 48) (end 141.015 48.015) (width 0.25) (layer "B.Cu") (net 24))
 (segment (start 95 89.08) (end 100.506167 89.08) (width 0.25) (layer "B.Cu") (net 24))
 (segment (start 156.355 48.015) (end 157.48 46.89) (width 0.25) (layer "B.Cu") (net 24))
 (segment (start 100.506167 89.08) (end 141 48.586167) (width 0.25) (layer "B.Cu") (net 24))
 (segment (start 141 48.586167) (end 141 48) (width 0.25) (layer "B.Cu") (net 24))
 (segment (start 170 51) (end 163.35 44.35) (width 0.25) (layer "F.Cu") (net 13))
 (segment (start 166.728299 80.125) (end 168.2 80.125) (width 0.25) (layer "F.Cu") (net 13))
 (segment (start 163.35 44.35) (end 157.48 44.35) (width 0.25) (layer "F.Cu") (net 13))
 (segment (start 165.85 87.935) (end 165.85 81.003299) (width 0.25) (layer "F.Cu") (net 13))
 (segment (start 165.85 81.003299) (end 166.728299 80.125) (width 0.25) (layer "F.Cu") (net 13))
 (segment (start 167.025 89.11) (end 165.85 87.935) (width 0.25) (layer "F.Cu") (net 13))
 (segment (start 168.2 80.125) (end 170 78.325) (width 0.25) (layer "F.Cu") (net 13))
 (segment (start 170 78.325) (end 170 51) (width 0.25) (layer "F.Cu") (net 13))
 (segment (start 100.999009 84) (end 141.999009 43) (width 0.25) (layer "B.Cu") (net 25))
 (segment (start 145.19 41.81) (end 157.48 41.81) (width 0.25) (layer "B.Cu") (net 25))
 (segment (start 95 84) (end 100.999009 84) (width 0.25) (layer "B.Cu") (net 25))
 (segment (start 144 43) (end 145.19 41.81) (width 0.25) (layer "B.Cu") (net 25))
 (segment (start 141.999009 43) (end 144 43) (width 0.25) (layer "B.Cu") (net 25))
 (segment (start 93.825 83.513299) (end 94.513299 82.825) (width 0.25) (layer "B.Cu") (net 26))
 (segment (start 156.355 40.395) (end 157.48 39.27) (width 0.25) (layer "B.Cu") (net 26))
 (segment (start 94.513299 82.825) (end 99.57 82.825) (width 0.25) (layer "B.Cu") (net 26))
 (segment (start 95 86.54) (end 93.825 85.365) (width 0.25) (layer "B.Cu") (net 26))
 (segment (start 93.825 85.365) (end 93.825 83.513299) (width 0.25) (layer "B.Cu") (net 26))
 (segment (start 99.57 82.825) (end 142 40.395) (width 0.25) (layer "B.Cu") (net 26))
 (segment (start 142 40.395) (end 156.355 40.395) (width 0.25) (layer "B.Cu") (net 26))
 (segment (start 171 80.055) (end 171 50) (width 0.25) (layer "F.Cu") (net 11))
 (segment (start 171 50) (end 170.75 50) (width 0.25) (layer "F.Cu") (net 11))
 (segment (start 170.75 50) (end 157.48 36.73) (width 0.25) (layer "F.Cu") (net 11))
 (segment (start 167.025 84.03) (end 171 80.055) (width 0.25) (layer "F.Cu") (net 11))
 (segment (start 173.586167 54.586167) (end 173 54) (width 0.25) (layer "F.Cu") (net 12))
 (segment (start 173.586167 80.008833) (end 173.586167 54.586167) (width 0.25) (layer "F.Cu") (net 12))
 (segment (start 167.025 86.57) (end 173.586167 80.008833) (width 0.25) (layer "F.Cu") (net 12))
 (segment (start 173 54) (end 173 49.71) (width 0.25) (layer "F.Cu") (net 12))
 (segment (start 173 49.71) (end 157.48 34.19) (width 0.25) (layer "F.Cu") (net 12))
 (segment (start 182.5 42.81) (end 172.81 42.81) (width 0.25) (layer "B.Cu") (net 29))
 (segment (start 172.81 42.81) (end 163 33) (width 0.25) (layer "B.Cu") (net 29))
 (segment (start 163 33) (end 165.76 30.24) (width 0.25) (layer "B.Cu") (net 29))
 (segment (start 165.76 30.24) (end 165.76 23.92) (width 0.25) (layer "B.Cu") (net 29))
 (segment (start 172.92 23.92) (end 170.84 23.92) (width 0.25) (layer "B.Cu") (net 3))
 (segment (start 183.25 34.25) (end 172.92 23.92) (width 0.25) (layer "B.Cu") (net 3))
 (segment (start 191.75 34.25) (end 183.25 34.25) (width 0.25) (layer "B.Cu") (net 3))
 (segment (start 115.544009 37.455991) (end 111.075 41.925) (width 0.25) (layer "B.Cu") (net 39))
 (segment (start 98.925 42.701167) (end 98.925 43.798833) (width 0.25) (layer "B.Cu") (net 39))
 (segment (start 98.925 43.798833) (end 100.151167 45.025) (width 0.25) (layer "B.Cu") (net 39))
 (segment (start 99.701167 41.925) (end 98.925 42.701167) (width 0.25) (layer "B.Cu") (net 39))
 (segment (start 100.151167 45.025) (end 103.025 45.025) (width 0.25) (layer "B.Cu") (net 39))
 (segment (start 104.075 46.075) (end 104.075 50.925) (width 0.25) (layer "B.Cu") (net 39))
 (segment (start 103.025 45.025) (end 104.075 46.075) (width 0.25) (layer "B.Cu") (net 39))
 (segment (start 104.075 50.925) (end 102.75 52.25) (width 0.25) (layer "B.Cu") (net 39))
 (segment (start 129 26) (end 129 23.84) (width 0.25) (layer "B.Cu") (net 39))
 (segment (start 125.489009 26) (end 115.544009 35.945) (width 0.25) (layer "B.Cu") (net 39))
 (segment (start 129 26) (end 125.489009 26) (width 0.25) (layer "B.Cu") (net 39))
 (segment (start 111.075 41.925) (end 99.701167 41.925) (width 0.25) (layer "B.Cu") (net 39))
 (segment (start 115.544009 35.945) (end 115.544009 37.455991) (width 0.25) (layer "B.Cu") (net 39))
 (segment (start 100 37) (end 110.84 37) (width 0.25) (layer "B.Cu") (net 30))
 (segment (start 93.75 43.25) (end 100 37) (width 0.25) (layer "B.Cu") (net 30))
 (segment (start 110.84 37) (end 124 23.84) (width 0.25) (layer "B.Cu") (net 30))
 (segment (start 130.125 23.125) (end 129.715 22.715) (width 0.25) (layer "B.Cu") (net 2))
 (segment (start 116.340991 43.25) (end 130.125 29.465991) (width 0.25) (layer "B.Cu") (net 2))
 (segment (start 129.715 22.715) (end 120.205 22.715) (width 0.25) (layer "B.Cu") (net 2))
 (segment (start 130.125 29.465991) (end 130.125 23.125) (width 0.25) (layer "B.Cu") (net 2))
 (segment (start 111.75 43.25) (end 116.340991 43.25) (width 0.25) (layer "B.Cu") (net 2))
 (segment (start 120.205 22.715) (end 119 23.92) (width 0.25) (layer "B.Cu") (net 2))
 (segment (start 132.425 22.265) (end 134 23.84) (width 0.25) (layer "B.Cu") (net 8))
 (segment (start 114.735 22.265) (end 132.425 22.265) (width 0.25) (layer "B.Cu") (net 8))
 (segment (start 102.75 34.25) (end 114.735 22.265) (width 0.25) (layer "B.Cu") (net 8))
 (segment (start 135.925 60.035) (end 132.75 63.21) (width 0.25) (layer "F.Cu") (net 35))
 (segment (start 145.705 60.035) (end 135.925 60.035) (width 0.25) (layer "F.Cu") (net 35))
 (segment (start 147.32 58.42) (end 145.705 60.035) (width 0.25) (layer "F.Cu") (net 35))
 (segment (start 155.96 58.42) (end 160.75 63.21) (width 0.25) (layer "F.Cu") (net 5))
 (segment (start 152.4 58.42) (end 155.96 58.42) (width 0.25) (layer "F.Cu") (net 5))
 (segment (start 177.045 25.045) (end 175.92 23.92) (width 0.25) (layer "B.Cu") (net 33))
 (segment (start 184.418833 25.045) (end 177.045 25.045) (width 0.25) (layer "B.Cu") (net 33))
 (segment (start 195 33) (end 192.373833 33) (width 0.25) (layer "B.Cu") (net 33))
 (segment (start 202.075 41.485) (end 202.075 36.201167) (width 0.25) (layer "B.Cu") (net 33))
 (segment (start 200.75 42.81) (end 202.075 41.485) (width 0.25) (layer "B.Cu") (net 33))
 (segment (start 192.373833 33) (end 184.418833 25.045) (width 0.25) (layer "B.Cu") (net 33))
 (segment (start 202.075 36.201167) (end 197.873833 32) (width 0.25) (layer "B.Cu") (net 33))
 (segment (start 197.873833 32) (end 196 32) (width 0.25) (layer "B.Cu") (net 33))
 (segment (start 196 32) (end 195 33) (width 0.25) (layer "B.Cu") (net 33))
 (segment (start 181 23.92) (end 183.825 26.745) (width 0.25) (layer "F.Cu") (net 32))
 (segment (start 183.825 43.325) (end 191.75 51.25) (width 0.25) (layer "F.Cu") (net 32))
 (segment (start 183.825 26.745) (end 183.825 43.325) (width 0.25) (layer "F.Cu") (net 32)))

